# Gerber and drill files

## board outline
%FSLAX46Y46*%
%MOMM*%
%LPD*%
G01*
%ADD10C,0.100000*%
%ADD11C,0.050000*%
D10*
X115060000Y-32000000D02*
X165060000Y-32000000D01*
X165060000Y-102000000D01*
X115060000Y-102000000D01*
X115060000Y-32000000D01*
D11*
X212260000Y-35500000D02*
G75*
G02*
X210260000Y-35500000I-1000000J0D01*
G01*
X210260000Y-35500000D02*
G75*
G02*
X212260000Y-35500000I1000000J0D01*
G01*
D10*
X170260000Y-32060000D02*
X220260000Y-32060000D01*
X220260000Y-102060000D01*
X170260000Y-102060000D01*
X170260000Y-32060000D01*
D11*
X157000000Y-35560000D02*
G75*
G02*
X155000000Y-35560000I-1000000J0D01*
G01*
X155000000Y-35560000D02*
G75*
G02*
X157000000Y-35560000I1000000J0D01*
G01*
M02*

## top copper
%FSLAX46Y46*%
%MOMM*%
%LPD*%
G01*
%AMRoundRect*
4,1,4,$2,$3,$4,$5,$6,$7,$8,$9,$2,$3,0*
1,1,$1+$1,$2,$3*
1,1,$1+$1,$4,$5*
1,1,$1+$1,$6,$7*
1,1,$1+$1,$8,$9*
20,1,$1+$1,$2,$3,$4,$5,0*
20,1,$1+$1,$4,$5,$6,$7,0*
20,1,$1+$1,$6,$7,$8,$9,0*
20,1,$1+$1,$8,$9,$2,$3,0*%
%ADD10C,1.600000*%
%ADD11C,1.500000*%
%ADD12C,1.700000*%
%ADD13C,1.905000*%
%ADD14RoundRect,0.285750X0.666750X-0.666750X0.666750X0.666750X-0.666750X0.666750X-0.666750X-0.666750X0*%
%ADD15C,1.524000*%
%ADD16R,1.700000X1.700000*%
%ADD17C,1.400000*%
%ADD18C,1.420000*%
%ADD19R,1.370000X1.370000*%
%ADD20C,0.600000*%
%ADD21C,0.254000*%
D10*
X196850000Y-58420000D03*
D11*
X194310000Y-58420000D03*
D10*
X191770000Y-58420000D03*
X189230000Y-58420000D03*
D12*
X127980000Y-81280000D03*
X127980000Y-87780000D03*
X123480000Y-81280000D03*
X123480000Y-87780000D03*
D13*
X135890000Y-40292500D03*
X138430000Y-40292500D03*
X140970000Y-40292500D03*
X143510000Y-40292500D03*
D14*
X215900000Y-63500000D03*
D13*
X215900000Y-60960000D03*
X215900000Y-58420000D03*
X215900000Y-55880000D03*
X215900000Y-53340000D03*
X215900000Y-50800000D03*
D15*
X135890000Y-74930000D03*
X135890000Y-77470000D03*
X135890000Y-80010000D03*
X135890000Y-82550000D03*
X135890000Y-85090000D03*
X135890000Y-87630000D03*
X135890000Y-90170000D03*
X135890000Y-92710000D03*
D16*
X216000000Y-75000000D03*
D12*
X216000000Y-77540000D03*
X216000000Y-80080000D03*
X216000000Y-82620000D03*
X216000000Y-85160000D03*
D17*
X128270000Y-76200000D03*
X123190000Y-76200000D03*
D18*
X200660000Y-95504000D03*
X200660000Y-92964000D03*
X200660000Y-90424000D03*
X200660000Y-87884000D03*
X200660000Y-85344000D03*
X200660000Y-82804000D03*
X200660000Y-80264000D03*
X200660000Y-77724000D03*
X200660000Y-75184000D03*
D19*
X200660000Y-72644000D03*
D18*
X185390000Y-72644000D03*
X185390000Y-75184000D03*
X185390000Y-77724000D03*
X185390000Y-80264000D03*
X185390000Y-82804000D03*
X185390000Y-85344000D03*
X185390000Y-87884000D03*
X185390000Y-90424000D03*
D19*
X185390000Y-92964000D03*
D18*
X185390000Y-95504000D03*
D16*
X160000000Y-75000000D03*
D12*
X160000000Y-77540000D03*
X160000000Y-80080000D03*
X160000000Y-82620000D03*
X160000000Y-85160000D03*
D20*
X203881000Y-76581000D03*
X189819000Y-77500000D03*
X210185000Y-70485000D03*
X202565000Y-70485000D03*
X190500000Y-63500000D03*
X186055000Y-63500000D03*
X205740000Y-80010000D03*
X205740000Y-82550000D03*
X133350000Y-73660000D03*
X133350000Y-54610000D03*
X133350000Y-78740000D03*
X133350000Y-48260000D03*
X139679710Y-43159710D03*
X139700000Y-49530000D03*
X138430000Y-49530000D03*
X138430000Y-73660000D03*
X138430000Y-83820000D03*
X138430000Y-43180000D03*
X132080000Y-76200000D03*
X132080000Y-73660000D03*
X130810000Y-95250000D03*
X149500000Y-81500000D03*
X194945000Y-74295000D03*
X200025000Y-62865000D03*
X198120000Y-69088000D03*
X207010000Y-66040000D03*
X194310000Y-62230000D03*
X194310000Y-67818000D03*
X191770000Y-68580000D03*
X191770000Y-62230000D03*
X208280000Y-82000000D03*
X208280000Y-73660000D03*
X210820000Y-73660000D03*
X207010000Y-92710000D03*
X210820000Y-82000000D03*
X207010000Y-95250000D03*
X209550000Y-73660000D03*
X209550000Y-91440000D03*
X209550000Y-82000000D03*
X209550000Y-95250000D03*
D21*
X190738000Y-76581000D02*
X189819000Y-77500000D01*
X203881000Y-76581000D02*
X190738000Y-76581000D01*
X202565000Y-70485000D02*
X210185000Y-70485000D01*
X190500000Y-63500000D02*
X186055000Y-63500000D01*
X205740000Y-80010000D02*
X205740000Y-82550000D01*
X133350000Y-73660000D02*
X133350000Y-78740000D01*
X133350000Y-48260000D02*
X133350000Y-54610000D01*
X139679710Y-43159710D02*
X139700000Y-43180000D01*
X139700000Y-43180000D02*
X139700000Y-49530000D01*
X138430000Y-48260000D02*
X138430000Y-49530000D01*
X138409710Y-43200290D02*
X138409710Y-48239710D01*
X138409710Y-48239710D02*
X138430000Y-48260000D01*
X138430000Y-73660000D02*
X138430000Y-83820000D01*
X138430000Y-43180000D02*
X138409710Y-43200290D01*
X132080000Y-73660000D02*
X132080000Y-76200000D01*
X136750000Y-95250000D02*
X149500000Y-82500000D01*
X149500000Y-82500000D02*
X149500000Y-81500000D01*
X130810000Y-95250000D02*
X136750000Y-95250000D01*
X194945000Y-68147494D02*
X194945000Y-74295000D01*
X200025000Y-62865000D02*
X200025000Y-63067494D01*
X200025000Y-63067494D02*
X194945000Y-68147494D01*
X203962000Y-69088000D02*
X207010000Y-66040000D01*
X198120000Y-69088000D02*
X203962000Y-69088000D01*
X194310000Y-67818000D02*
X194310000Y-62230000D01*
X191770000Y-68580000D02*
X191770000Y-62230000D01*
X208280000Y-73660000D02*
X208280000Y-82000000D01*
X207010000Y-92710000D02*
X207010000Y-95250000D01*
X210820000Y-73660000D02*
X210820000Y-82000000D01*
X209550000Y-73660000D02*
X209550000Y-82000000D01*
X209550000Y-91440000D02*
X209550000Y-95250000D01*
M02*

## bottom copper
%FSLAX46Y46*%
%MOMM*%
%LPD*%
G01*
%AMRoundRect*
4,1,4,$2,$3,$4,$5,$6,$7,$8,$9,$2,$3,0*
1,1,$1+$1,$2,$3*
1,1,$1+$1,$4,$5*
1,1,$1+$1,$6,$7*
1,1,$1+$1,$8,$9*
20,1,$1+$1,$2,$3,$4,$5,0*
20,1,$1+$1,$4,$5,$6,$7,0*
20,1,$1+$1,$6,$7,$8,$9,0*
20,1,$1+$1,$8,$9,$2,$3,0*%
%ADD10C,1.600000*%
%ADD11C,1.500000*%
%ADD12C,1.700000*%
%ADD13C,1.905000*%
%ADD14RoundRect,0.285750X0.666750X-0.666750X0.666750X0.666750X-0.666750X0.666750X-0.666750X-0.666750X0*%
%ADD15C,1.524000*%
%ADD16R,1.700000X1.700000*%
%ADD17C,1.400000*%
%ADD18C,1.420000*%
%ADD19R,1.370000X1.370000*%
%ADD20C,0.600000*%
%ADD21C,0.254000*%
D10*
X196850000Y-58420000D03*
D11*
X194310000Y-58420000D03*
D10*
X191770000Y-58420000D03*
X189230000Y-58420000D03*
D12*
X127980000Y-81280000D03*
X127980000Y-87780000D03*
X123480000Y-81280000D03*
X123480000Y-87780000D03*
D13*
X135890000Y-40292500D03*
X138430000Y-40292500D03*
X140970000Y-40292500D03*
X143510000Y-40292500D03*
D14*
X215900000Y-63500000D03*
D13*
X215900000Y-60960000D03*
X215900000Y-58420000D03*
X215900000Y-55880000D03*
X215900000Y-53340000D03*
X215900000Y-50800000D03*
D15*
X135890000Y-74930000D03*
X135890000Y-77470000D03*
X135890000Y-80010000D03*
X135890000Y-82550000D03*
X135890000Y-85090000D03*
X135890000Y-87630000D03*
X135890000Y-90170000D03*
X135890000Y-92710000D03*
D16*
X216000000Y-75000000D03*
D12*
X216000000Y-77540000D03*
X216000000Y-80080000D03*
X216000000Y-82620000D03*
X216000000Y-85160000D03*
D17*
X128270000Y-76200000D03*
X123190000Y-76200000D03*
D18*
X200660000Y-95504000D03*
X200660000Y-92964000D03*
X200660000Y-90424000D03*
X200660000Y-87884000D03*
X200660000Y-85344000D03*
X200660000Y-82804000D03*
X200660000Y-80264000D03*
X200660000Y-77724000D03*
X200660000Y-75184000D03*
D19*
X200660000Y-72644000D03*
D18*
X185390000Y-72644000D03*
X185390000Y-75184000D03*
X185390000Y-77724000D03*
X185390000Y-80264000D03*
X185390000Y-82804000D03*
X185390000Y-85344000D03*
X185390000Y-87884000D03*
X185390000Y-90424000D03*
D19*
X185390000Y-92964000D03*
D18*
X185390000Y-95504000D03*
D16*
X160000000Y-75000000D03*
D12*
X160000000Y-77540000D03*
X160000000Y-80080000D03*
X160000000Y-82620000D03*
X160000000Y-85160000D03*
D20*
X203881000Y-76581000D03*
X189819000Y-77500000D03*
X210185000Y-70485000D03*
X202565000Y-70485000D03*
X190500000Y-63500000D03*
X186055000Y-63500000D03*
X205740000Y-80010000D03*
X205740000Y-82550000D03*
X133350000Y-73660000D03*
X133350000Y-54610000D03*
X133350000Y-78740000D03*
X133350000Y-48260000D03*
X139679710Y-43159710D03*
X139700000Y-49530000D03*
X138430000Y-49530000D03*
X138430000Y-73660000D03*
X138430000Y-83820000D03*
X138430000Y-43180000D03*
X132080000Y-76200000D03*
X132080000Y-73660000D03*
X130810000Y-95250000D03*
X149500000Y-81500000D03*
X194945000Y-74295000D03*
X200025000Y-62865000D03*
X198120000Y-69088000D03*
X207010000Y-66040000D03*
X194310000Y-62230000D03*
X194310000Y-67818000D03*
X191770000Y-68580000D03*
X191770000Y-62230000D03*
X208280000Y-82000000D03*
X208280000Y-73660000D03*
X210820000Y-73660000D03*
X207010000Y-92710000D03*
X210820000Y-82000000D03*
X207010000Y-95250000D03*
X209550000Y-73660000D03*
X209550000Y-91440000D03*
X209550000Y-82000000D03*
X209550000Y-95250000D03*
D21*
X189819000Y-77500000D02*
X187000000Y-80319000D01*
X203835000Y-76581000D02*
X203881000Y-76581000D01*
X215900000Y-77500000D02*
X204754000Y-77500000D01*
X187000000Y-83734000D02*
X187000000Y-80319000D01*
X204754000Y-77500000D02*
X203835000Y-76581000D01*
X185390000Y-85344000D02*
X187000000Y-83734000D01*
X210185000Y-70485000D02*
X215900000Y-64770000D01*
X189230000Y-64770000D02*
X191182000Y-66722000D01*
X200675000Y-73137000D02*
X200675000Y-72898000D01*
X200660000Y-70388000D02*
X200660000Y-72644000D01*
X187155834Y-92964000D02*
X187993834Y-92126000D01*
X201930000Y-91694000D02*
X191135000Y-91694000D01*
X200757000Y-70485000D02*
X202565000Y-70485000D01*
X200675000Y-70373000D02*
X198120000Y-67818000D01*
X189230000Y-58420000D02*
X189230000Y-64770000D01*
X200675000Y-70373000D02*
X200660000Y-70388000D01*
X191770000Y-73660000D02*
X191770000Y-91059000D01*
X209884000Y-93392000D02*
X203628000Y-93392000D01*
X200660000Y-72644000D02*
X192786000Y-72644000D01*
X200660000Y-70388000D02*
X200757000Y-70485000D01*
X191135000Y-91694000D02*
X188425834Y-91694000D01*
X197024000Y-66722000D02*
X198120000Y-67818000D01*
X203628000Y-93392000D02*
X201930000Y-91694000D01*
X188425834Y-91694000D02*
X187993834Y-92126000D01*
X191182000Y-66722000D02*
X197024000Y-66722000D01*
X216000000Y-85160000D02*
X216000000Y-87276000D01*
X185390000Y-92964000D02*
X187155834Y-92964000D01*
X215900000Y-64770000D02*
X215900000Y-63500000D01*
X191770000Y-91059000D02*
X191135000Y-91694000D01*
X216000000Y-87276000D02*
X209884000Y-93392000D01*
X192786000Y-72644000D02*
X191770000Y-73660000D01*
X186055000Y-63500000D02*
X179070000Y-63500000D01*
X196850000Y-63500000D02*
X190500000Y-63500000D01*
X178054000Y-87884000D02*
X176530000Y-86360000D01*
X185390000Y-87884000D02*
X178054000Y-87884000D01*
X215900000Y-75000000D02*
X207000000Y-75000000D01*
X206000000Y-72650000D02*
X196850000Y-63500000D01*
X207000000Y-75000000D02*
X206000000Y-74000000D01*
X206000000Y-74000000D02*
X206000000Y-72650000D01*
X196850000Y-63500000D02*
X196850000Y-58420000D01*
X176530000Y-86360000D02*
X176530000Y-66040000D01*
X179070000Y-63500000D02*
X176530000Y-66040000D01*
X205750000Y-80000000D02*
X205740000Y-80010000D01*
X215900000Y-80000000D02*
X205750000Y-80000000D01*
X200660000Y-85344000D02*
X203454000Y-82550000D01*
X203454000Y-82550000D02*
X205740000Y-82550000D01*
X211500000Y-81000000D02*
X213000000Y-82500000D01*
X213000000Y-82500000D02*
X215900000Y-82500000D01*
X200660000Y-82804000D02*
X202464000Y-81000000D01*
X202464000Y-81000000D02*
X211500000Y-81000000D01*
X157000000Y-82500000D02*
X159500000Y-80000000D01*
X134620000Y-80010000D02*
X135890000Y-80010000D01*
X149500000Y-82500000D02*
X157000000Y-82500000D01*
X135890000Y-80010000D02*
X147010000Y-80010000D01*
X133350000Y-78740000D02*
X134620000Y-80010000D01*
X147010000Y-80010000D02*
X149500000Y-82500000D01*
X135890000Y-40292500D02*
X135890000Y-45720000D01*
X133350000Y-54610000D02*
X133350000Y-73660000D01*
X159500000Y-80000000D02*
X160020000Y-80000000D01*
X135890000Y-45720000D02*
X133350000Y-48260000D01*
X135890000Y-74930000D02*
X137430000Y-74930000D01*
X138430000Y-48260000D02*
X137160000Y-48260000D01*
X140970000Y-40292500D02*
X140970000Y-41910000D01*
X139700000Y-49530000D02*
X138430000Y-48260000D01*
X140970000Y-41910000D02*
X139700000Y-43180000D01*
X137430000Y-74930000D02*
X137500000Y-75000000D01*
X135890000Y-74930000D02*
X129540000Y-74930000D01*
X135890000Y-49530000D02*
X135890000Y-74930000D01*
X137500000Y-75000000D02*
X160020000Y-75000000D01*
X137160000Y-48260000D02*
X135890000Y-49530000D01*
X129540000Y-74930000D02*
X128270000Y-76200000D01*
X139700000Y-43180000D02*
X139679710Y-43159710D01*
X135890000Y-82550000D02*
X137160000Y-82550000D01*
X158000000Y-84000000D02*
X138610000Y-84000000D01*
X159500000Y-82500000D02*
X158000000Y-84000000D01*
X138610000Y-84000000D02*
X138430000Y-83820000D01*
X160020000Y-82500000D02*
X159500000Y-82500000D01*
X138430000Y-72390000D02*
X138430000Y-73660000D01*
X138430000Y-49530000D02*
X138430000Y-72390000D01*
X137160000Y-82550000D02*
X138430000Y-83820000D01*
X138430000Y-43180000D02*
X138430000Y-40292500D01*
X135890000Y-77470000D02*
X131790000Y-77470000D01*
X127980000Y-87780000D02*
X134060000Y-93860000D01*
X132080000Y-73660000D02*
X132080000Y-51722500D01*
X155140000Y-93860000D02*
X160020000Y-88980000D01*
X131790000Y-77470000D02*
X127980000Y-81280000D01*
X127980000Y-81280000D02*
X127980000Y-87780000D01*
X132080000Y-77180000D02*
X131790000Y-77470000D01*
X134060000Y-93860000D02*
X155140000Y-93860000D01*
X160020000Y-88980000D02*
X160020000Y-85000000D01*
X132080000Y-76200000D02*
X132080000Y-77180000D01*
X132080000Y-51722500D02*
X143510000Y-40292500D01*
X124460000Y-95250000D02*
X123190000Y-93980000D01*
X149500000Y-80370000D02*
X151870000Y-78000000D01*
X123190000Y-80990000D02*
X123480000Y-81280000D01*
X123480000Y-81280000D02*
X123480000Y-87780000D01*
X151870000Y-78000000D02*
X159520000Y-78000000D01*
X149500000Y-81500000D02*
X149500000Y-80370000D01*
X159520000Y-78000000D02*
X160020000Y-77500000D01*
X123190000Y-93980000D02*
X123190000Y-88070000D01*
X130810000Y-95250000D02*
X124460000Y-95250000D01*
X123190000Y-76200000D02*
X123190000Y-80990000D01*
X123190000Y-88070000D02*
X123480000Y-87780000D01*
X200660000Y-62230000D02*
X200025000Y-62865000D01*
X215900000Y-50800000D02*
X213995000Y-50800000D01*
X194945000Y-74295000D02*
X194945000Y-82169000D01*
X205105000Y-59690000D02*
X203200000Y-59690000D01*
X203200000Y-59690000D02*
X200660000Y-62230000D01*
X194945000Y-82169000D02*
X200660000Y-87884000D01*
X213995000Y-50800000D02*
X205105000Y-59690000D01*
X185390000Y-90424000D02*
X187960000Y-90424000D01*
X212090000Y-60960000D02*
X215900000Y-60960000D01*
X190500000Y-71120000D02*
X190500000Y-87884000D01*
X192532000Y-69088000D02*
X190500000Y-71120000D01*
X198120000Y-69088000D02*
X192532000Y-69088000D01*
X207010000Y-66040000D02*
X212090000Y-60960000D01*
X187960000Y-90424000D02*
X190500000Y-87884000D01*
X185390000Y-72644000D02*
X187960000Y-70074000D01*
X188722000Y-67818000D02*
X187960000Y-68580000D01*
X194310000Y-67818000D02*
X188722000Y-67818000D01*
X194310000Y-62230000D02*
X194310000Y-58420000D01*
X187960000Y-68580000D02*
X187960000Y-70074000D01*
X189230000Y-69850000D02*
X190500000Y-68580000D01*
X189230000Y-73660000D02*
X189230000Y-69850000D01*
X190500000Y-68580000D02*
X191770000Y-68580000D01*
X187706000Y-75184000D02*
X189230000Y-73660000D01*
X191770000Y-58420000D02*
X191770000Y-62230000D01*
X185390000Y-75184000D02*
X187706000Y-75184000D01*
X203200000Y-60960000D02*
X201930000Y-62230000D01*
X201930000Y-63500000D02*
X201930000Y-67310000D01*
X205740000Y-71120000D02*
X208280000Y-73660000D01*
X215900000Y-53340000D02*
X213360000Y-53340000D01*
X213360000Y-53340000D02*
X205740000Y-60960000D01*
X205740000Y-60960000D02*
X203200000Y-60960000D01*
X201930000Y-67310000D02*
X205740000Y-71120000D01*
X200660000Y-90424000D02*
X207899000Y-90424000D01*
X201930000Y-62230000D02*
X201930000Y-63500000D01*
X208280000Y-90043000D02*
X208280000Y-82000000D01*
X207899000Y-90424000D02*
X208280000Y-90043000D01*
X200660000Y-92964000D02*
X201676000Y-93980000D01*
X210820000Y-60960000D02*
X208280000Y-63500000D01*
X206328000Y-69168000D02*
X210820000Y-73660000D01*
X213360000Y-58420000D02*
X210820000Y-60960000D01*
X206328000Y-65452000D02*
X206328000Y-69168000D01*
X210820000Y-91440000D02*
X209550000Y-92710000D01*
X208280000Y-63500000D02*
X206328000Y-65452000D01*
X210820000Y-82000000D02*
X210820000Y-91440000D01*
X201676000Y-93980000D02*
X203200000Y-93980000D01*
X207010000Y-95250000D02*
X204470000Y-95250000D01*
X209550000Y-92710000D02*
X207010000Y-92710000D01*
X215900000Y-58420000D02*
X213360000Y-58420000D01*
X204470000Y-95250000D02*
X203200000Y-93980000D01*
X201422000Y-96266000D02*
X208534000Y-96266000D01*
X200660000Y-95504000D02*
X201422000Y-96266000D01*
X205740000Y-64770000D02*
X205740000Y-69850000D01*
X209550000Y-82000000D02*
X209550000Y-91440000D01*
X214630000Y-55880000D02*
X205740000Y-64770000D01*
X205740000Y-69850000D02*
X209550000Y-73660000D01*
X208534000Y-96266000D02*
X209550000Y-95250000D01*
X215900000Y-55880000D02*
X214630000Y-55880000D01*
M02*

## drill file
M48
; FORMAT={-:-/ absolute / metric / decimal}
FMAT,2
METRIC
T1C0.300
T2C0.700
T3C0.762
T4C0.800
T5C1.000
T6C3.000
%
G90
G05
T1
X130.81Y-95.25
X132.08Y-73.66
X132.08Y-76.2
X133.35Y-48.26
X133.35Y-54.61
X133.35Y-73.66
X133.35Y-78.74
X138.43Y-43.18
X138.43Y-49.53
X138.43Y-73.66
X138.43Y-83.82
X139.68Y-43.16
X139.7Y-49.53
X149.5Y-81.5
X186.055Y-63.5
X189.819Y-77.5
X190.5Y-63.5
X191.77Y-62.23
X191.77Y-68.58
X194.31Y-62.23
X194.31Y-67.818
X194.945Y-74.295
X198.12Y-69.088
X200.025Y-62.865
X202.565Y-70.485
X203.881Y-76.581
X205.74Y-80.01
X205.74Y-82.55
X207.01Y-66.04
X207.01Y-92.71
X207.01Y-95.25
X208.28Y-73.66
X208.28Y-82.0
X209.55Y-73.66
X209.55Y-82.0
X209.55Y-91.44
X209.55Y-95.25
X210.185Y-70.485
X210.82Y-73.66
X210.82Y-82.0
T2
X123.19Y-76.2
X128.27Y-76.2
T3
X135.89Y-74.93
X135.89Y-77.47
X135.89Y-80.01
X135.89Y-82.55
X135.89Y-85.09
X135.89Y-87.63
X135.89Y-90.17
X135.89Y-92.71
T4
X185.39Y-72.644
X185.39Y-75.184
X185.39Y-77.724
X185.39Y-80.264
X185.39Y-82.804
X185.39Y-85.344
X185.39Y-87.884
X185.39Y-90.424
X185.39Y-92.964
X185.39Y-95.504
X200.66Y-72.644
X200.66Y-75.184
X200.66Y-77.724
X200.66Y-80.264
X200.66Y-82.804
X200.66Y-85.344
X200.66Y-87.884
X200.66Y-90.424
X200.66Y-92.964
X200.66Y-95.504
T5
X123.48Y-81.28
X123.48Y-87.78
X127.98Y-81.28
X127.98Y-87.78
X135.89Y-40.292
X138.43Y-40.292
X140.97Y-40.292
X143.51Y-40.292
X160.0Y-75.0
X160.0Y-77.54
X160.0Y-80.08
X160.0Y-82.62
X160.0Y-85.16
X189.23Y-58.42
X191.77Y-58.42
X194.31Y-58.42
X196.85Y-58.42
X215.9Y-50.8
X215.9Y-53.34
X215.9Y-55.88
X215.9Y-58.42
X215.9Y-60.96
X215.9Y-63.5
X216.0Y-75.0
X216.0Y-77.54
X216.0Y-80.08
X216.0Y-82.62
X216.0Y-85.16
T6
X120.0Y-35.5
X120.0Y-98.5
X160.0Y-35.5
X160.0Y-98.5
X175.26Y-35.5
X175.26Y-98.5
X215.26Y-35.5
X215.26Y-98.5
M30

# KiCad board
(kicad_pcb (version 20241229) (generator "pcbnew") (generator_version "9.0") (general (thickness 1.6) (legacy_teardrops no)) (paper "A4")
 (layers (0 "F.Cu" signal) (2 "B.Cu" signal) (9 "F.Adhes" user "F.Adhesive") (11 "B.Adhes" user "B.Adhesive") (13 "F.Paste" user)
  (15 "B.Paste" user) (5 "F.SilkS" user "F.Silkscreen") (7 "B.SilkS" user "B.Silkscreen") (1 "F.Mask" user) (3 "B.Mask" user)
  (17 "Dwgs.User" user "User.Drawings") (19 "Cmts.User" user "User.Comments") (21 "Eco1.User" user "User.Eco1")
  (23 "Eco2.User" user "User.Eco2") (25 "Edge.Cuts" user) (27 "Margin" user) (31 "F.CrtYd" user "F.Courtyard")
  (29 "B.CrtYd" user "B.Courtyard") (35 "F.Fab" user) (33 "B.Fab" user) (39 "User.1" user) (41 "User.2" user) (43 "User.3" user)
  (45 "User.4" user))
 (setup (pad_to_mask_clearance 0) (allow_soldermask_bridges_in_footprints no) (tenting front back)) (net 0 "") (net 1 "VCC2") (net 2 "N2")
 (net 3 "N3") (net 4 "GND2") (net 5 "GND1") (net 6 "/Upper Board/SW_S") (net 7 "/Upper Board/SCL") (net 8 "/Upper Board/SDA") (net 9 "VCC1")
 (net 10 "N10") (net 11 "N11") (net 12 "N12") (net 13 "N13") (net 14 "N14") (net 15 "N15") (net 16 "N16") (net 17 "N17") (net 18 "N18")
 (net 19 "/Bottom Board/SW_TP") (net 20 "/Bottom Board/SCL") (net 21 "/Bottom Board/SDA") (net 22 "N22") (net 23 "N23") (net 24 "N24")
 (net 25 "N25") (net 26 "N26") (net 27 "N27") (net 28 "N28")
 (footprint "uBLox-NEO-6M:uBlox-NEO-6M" (layer "F.Cu") (at 193.04 43.18 180)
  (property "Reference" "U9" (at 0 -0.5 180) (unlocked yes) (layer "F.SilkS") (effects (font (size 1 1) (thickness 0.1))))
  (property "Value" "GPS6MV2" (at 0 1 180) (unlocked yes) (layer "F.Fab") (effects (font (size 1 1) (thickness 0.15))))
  (pad "1" thru_hole circle (at -3.81 -15.24 180) (size 1.6 1.6) (drill 1) (layers "*.Cu" "*.Mask") (remove_unused_layers no) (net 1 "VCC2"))
  (pad "2" thru_hole circle (at -1.27 -15.24 180) (size 1.5 1.5) (drill 1) (layers "*.Cu" "F.Mask" "F.Paste") (remove_unused_layers no)
   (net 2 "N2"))
  (pad "3" thru_hole circle (at 1.27 -15.24 180) (size 1.6 1.6) (drill 1) (layers "*.Cu" "F.Mask" "F.Paste") (remove_unused_layers no)
   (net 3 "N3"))
  (pad "4" thru_hole circle (at 3.81 -15.24 180) (size 1.6 1.6) (drill 1) (layers "*.Cu" "F.Mask" "F.Paste") (remove_unused_layers no)
   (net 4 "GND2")))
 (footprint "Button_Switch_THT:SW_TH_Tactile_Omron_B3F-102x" (layer "F.Cu") (at 127.98 81.28 -90)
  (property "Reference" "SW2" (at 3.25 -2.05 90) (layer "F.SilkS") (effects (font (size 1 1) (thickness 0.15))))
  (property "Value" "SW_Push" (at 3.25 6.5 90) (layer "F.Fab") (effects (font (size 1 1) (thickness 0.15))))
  (pad "1" thru_hole circle (at 0 0 270) (size 1.7 1.7) (drill 1) (layers "*.Cu" "*.Mask") (remove_unused_layers no) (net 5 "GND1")
   (thermal_bridge_angle 90))
  (pad "1" thru_hole circle (at 6.5 0 270) (size 1.7 1.7) (drill 1) (layers "*.Cu" "*.Mask") (remove_unused_layers no) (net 5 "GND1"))
  (pad "2" thru_hole circle (at 0 4.5 270) (size 1.7 1.7) (drill 1) (layers "*.Cu" "*.Mask") (remove_unused_layers no)
   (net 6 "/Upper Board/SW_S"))
  (pad "2" thru_hole circle (at 6.5 4.5 270) (size 1.7 1.7) (drill 1) (layers "*.Cu" "*.Mask") (remove_unused_layers no)
   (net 6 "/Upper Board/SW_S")))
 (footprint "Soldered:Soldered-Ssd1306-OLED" (layer "F.Cu") (at 139.7 40.2925)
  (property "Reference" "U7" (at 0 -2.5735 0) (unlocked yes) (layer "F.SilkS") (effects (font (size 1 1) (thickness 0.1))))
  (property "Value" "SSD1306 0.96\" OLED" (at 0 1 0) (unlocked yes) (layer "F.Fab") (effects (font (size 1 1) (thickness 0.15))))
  (pad "1" thru_hole circle (at -3.81 0) (size 1.905 1.905) (drill 1) (layers "*.Cu" "*.Mask") (remove_unused_layers no)
   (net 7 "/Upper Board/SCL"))
  (pad "2" thru_hole circle (at -1.27 0) (size 1.905 1.905) (drill 1) (layers "*.Cu" "*.Mask") (remove_unused_layers no)
   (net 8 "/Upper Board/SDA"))
  (pad "3" thru_hole circle (at 1.27 0) (size 1.905 1.905) (drill 1) (layers "*.Cu" "*.Mask") (remove_unused_layers no) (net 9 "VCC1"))
  (pad "4" thru_hole circle (at 3.81 0) (size 1.905 1.905) (drill 1) (layers "*.Cu" "*.Mask") (remove_unused_layers no) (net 5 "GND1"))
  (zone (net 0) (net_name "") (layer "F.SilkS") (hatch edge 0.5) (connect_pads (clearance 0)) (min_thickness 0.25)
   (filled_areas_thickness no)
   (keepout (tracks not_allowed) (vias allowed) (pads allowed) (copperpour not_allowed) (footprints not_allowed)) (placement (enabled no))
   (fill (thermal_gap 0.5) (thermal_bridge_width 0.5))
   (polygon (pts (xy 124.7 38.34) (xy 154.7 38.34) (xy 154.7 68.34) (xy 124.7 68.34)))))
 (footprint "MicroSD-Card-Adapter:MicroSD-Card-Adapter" (layer "F.Cu") (at 215.9 57.2008 90)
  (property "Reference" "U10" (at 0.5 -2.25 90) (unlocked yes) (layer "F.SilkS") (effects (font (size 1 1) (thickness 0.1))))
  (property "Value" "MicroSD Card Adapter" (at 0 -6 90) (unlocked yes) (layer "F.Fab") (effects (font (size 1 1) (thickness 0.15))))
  (pad "1" thru_hole roundrect (at -6.2992 0 90) (size 1.905 1.905) (drill 1) (layers "*.Cu" "*.Mask") (remove_unused_layers no)
   (roundrect_rratio 0.15) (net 4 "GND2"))
  (pad "2" thru_hole circle (at -3.7592 0 90) (size 1.905 1.905) (drill 1) (layers "*.Cu" "*.Mask") (remove_unused_layers no) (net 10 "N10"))
  (pad "3" thru_hole circle (at -1.2192 0 90) (size 1.905 1.905) (drill 1) (layers "*.Cu" "*.Mask") (remove_unused_layers no) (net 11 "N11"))
  (pad "4" thru_hole circle (at 1.3208 0 90) (size 1.905 1.905) (drill 1) (layers "*.Cu" "*.Mask") (remove_unused_layers no) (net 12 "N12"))
  (pad "5" thru_hole circle (at 3.8608 0 90) (size 1.905 1.905) (drill 1) (layers "*.Cu" "*.Mask") (remove_unused_layers no) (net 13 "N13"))
  (pad "6" thru_hole circle (at 6.4008 0 90) (size 1.905 1.905) (drill 1) (layers "*.Cu" "*.Mask") (remove_unused_layers no) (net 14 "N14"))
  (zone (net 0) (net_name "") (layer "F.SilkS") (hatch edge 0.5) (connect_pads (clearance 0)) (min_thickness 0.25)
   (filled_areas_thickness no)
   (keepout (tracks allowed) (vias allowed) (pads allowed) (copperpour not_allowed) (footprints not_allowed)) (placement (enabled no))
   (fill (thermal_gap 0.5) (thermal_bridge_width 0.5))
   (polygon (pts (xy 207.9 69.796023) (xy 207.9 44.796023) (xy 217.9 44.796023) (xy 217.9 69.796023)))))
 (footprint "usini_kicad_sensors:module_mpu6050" (layer "F.Cu") (at 135.89 92.71)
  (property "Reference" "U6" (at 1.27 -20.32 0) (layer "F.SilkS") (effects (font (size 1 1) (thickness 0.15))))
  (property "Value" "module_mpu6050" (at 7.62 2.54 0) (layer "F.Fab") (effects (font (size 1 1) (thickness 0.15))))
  (pad "1" thru_hole circle (at 0 -17.78) (size 1.524 1.524) (drill 0.762) (layers "*.Cu" "*.Mask") (remove_unused_layers no) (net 9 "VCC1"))
  (pad "2" thru_hole circle (at 0 -15.24) (size 1.524 1.524) (drill 0.762) (layers "*.Cu" "*.Mask") (remove_unused_layers no) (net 5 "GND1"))
  (pad "3" thru_hole circle (at 0 -12.7) (size 1.524 1.524) (drill 0.762) (layers "*.Cu" "*.Mask") (remove_unused_layers no)
   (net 7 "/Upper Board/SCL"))
  (pad "4" thru_hole circle (at 0 -10.16) (size 1.524 1.524) (drill 0.762) (layers "*.Cu" "*.Mask") (remove_unused_layers no)
   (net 8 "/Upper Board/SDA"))
  (pad "5" thru_hole circle (at 0 -7.62) (size 1.524 1.524) (drill 0.762) (layers "*.Cu" "*.Mask") (remove_unused_layers no) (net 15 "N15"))
  (pad "6" thru_hole circle (at 0 -5.08) (size 1.524 1.524) (drill 0.762) (layers "*.Cu" "*.Mask") (remove_unused_layers no) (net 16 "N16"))
  (pad "7" thru_hole circle (at 0 -2.54) (size 1.524 1.524) (drill 0.762) (layers "*.Cu" "*.Mask") (remove_unused_layers no) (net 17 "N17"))
  (pad "8" thru_hole circle (at 0 0) (size 1.524 1.524) (drill 0.762) (layers "*.Cu" "*.Mask") (remove_unused_layers no) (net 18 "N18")))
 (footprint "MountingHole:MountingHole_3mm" (layer "F.Cu") (at 215.26 98.5)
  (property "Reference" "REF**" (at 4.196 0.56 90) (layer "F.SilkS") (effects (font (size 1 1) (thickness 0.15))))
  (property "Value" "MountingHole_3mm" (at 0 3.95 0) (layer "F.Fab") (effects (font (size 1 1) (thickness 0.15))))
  (pad "" np_thru_hole circle (at 0 0) (size 3 3) (drill 3) (layers "*.Cu" "*.Mask")))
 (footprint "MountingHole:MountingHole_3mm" (layer "F.Cu") (at 160 98.5)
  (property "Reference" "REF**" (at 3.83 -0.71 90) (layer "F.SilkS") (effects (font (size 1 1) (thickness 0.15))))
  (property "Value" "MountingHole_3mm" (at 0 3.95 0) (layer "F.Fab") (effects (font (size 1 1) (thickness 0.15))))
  (pad "" np_thru_hole circle (at 0 0) (size 3 3) (drill 3) (layers "*.Cu" "*.Mask")))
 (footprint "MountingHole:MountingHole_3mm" (layer "F.Cu") (at 175.26 98.5)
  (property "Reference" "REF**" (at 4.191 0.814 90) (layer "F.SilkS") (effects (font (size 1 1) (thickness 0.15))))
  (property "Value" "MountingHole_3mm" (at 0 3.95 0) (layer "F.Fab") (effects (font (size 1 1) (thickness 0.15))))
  (pad "" np_thru_hole circle (at 0 0) (size 3 3) (drill 3) (layers "*.Cu" "*.Mask")))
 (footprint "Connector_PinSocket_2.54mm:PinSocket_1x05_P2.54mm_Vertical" (layer "F.Cu") (at 216 75)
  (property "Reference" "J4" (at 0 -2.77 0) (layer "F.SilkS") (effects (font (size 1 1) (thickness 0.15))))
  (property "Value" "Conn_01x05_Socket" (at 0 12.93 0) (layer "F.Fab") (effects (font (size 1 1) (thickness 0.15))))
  (pad "1" thru_hole rect (at 0 0) (size 1.7 1.7) (drill 1) (layers "*.Cu" "*.Mask") (remove_unused_layers no) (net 1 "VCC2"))
  (pad "2" thru_hole circle (at 0 2.54) (size 1.7 1.7) (drill 1) (layers "*.Cu" "*.Mask") (remove_unused_layers no)
   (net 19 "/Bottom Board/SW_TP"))
  (pad "3" thru_hole circle (at 0 5.08) (size 1.7 1.7) (drill 1) (layers "*.Cu" "*.Mask") (remove_unused_layers no)
   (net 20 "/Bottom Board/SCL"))
  (pad "4" thru_hole circle (at 0 7.62) (size 1.7 1.7) (drill 1) (layers "*.Cu" "*.Mask") (remove_unused_layers no)
   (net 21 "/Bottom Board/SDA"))
  (pad "5" thru_hole circle (at 0 10.16) (size 1.7 1.7) (drill 1) (layers "*.Cu" "*.Mask") (remove_unused_layers no) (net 4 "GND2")))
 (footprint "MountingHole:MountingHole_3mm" (layer "F.Cu") (at 215.26 35.5)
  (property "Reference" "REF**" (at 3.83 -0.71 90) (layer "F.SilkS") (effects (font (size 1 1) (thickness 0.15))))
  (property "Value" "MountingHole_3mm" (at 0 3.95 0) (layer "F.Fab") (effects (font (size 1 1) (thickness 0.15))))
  (pad "" np_thru_hole circle (at 0 0) (size 3 3) (drill 3) (layers "*.Cu" "*.Mask")))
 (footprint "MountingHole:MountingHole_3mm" (layer "F.Cu") (at 120 35.5)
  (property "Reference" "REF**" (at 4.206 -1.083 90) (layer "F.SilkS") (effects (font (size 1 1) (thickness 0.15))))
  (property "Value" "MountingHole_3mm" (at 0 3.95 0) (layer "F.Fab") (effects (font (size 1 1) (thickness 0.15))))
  (pad "" np_thru_hole circle (at 0 0) (size 3 3) (drill 3) (layers "*.Cu" "*.Mask")))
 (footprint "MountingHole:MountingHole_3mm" (layer "F.Cu") (at 175.26 35.5)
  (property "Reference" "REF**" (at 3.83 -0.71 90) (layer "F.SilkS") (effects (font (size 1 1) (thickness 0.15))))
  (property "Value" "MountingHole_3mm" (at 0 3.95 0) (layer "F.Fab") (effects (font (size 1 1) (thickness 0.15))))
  (pad "" np_thru_hole circle (at 0 0) (size 3 3) (drill 3) (layers "*.Cu" "*.Mask")))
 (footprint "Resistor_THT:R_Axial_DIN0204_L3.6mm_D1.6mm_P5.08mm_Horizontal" (layer "F.Cu") (at 128.27 76.2 180)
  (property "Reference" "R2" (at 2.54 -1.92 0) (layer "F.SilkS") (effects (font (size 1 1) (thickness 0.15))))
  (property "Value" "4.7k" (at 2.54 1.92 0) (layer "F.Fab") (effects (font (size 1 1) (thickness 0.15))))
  (pad "1" thru_hole circle (at 0 0 180) (size 1.4 1.4) (drill 0.7) (layers "*.Cu" "*.Mask") (remove_unused_layers no) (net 9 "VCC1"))
  (pad "2" thru_hole circle (at 5.08 0 180) (size 1.4 1.4) (drill 0.7) (layers "*.Cu" "*.Mask") (remove_unused_layers no)
   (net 6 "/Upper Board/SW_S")))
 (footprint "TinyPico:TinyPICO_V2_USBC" (layer "F.Cu") (at 193.025 84.074 180)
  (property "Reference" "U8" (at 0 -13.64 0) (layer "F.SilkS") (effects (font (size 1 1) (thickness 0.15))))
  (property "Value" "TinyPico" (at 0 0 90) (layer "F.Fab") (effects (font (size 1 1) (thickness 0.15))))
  (pad "1" thru_hole circle (at -7.635 -11.43 90) (size 1.42 1.42) (drill 0.8) (layers "*.Cu" "*.Mask") (remove_unused_layers no)
   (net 12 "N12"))
  (pad "2" thru_hole circle (at -7.635 -8.89 90) (size 1.42 1.42) (drill 0.8) (layers "*.Cu" "*.Mask") (remove_unused_layers no)
   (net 11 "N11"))
  (pad "3" thru_hole circle (at -7.635 -6.35 90) (size 1.42 1.42) (drill 0.8) (layers "*.Cu" "*.Mask") (remove_unused_layers no)
   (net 13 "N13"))
  (pad "4" thru_hole circle (at -7.635 -3.81 90) (size 1.42 1.42) (drill 0.8) (layers "*.Cu" "*.Mask") (remove_unused_layers no)
   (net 14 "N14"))
  (pad "5" thru_hole circle (at -7.635 -1.27 90) (size 1.42 1.42) (drill 0.8) (layers "*.Cu" "*.Mask") (remove_unused_layers no)
   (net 20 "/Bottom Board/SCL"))
  (pad "6" thru_hole circle (at -7.635 1.27 90) (size 1.42 1.42) (drill 0.8) (layers "*.Cu" "*.Mask") (remove_unused_layers no)
   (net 21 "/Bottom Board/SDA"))
  (pad "7" thru_hole circle (at -7.635 3.81 90) (size 1.42 1.42) (drill 0.8) (layers "*.Cu" "*.Mask") (remove_unused_layers no)
   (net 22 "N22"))
  (pad "8" thru_hole circle (at -7.635 6.35 90) (size 1.42 1.42) (drill 0.8) (layers "*.Cu" "*.Mask") (remove_unused_layers no)
   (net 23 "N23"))
  (pad "9" thru_hole circle (at -7.635 8.89 90) (size 1.42 1.42) (drill 0.8) (layers "*.Cu" "*.Mask") (remove_unused_layers no)
   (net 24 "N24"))
  (pad "10" thru_hole rect (at -7.635 11.43 90) (size 1.37 1.37) (drill 0.8) (layers "*.Cu" "*.Mask") (remove_unused_layers no)
   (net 4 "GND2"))
  (pad "11" thru_hole circle (at 7.635 11.43 90) (size 1.42 1.42) (drill 0.8) (layers "*.Cu" "*.Mask") (remove_unused_layers no)
   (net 2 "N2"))
  (pad "12" thru_hole circle (at 7.635 8.89 90) (size 1.42 1.42) (drill 0.8) (layers "*.Cu" "*.Mask") (remove_unused_layers no) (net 3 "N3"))
  (pad "13" thru_hole circle (at 7.635 6.35 90) (size 1.42 1.42) (drill 0.8) (layers "*.Cu" "*.Mask") (remove_unused_layers no)
   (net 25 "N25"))
  (pad "14" thru_hole circle (at 7.635 3.81 90) (size 1.42 1.42) (drill 0.8) (layers "*.Cu" "*.Mask") (remove_unused_layers no)
   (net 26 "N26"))
  (pad "15" thru_hole circle (at 7.635 1.27 90) (size 1.42 1.42) (drill 0.8) (layers "*.Cu" "*.Mask") (remove_unused_layers no)
   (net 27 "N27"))
  (pad "16" thru_hole circle (at 7.635 -1.27 90) (size 1.42 1.42) (drill 0.8) (layers "*.Cu" "*.Mask") (remove_unused_layers no)
   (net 19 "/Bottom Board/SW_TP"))
  (pad "17" thru_hole circle (at 7.635 -3.81 90) (size 1.42 1.42) (drill 0.8) (layers "*.Cu" "*.Mask") (remove_unused_layers no)
   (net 1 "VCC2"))
  (pad "18" thru_hole circle (at 7.635 -6.35 90) (size 1.42 1.42) (drill 0.8) (layers "*.Cu" "*.Mask") (remove_unused_layers no)
   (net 10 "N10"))
  (pad "19" thru_hole rect (at 7.635 -8.89 90) (size 1.37 1.37) (drill 0.8) (layers "*.Cu" "*.Mask") (remove_unused_layers no)
   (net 4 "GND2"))
  (pad "20" thru_hole circle (at 7.635 -11.43 90) (size 1.42 1.42) (drill 0.8) (layers "*.Cu" "*.Mask") (remove_unused_layers no)
   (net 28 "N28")))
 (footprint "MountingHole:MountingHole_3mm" (layer "F.Cu") (at 120 98.5)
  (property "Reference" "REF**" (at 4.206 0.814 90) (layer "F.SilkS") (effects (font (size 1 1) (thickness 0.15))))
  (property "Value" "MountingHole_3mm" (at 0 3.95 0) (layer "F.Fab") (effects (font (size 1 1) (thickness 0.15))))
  (pad "" np_thru_hole circle (at 0 0) (size 3 3) (drill 3) (layers "*.Cu" "*.Mask")))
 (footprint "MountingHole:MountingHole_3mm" (layer "F.Cu") (at 160 35.5)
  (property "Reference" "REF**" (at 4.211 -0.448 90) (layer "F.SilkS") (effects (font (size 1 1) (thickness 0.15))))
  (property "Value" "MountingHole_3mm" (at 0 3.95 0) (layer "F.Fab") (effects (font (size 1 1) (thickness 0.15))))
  (pad "" np_thru_hole circle (at 0 0) (size 3 3) (drill 3) (layers "*.Cu" "*.Mask")))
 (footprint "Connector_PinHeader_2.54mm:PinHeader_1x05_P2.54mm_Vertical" (layer "B.Cu") (at 160 75 180)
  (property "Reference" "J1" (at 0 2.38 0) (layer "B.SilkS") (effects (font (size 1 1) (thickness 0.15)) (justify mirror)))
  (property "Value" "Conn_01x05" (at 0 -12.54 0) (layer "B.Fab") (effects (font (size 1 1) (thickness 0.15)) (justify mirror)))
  (pad "1" thru_hole rect (at 0 0 180) (size 1.7 1.7) (drill 1) (layers "*.Cu" "*.Mask") (remove_unused_layers no) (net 9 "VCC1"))
  (pad "2" thru_hole circle (at 0 -2.54 180) (size 1.7 1.7) (drill 1) (layers "*.Cu" "*.Mask") (remove_unused_layers no)
   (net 6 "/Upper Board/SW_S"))
  (pad "3" thru_hole circle (at 0 -5.08 180) (size 1.7 1.7) (drill 1) (layers "*.Cu" "*.Mask") (remove_unused_layers no)
   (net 7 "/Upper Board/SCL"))
  (pad "4" thru_hole circle (at 0 -7.62 180) (size 1.7 1.7) (drill 1) (layers "*.Cu" "*.Mask") (remove_unused_layers no)
   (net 8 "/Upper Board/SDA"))
  (pad "5" thru_hole circle (at 0 -10.16 180) (size 1.7 1.7) (drill 1) (layers "*.Cu" "*.Mask") (remove_unused_layers no) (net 5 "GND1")))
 (gr_rect (start 115.06 32) (end 165.06 102) (stroke (width 0.1) (type solid)) (fill no) (layer "Edge.Cuts"))
 (gr_circle (center 211.26 35.5) (end 212.26 35.5) (stroke (width 0.05) (type solid)) (fill no) (layer "Edge.Cuts"))
 (gr_rect (start 170.26 32.06) (end 220.26 102.06) (stroke (width 0.1) (type solid)) (fill no) (layer "Edge.Cuts"))
 (gr_circle (center 156 35.56) (end 157 35.56) (stroke (width 0.05) (type solid)) (fill no) (layer "Edge.Cuts"))
 (segment (start 190.738 76.581) (end 189.819 77.5) (width 0.254) (layer "F.Cu") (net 19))
 (segment (start 203.881 76.581) (end 190.738 76.581) (width 0.254) (layer "F.Cu") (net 19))
 (via (at 203.881 76.581) (size 0.6) (drill 0.3) (layers "F.Cu" "B.Cu") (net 19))
 (via (at 189.819 77.5) (size 0.6) (drill 0.3) (layers "F.Cu" "B.Cu") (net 19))
 (segment (start 189.819 77.5) (end 187 80.319) (width 0.254) (layer "B.Cu") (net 19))
 (segment (start 203.835 76.581) (end 203.881 76.581) (width 0.254) (layer "B.Cu") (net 19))
 (segment (start 215.9 77.5) (end 204.754 77.5) (width 0.254) (layer "B.Cu") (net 19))
 (segment (start 187 83.734) (end 187 80.319) (width 0.254) (layer "B.Cu") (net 19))
 (segment (start 204.754 77.5) (end 203.835 76.581) (width 0.254) (layer "B.Cu") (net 19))
 (segment (start 185.39 85.344) (end 187 83.734) (width 0.254) (layer "B.Cu") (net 19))
 (segment (start 202.565 70.485) (end 210.185 70.485) (width 0.254) (layer "F.Cu") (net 4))
 (via (at 210.185 70.485) (size 0.6) (drill 0.3) (layers "F.Cu" "B.Cu") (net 4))
 (via (at 202.565 70.485) (size 0.6) (drill 0.3) (layers "F.Cu" "B.Cu") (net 4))
 (segment (start 210.185 70.485) (end 215.9 64.77) (width 0.254) (layer "B.Cu") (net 4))
 (segment (start 189.23 64.77) (end 191.182 66.722) (width 0.254) (layer "B.Cu") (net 4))
 (segment (start 200.675 73.137) (end 200.675 72.898) (width 0.254) (layer "B.Cu") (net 4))
 (segment (start 200.66 70.388) (end 200.66 72.644) (width 0.254) (layer "B.Cu") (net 4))
 (segment (start 187.155834 92.964) (end 187.993834 92.126) (width 0.254) (layer "B.Cu") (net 4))
 (segment (start 201.93 91.694) (end 191.135 91.694) (width 0.254) (layer "B.Cu") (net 4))
 (segment (start 200.757 70.485) (end 202.565 70.485) (width 0.254) (layer "B.Cu") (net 4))
 (segment (start 200.675 70.373) (end 198.12 67.818) (width 0.254) (layer "B.Cu") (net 4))
 (segment (start 189.23 58.42) (end 189.23 64.77) (width 0.254) (layer "B.Cu") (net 4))
 (segment (start 200.675 70.373) (end 200.66 70.388) (width 0.254) (layer "B.Cu") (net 4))
 (segment (start 191.77 73.66) (end 191.77 91.059) (width 0.254) (layer "B.Cu") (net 4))
 (segment (start 209.884 93.392) (end 203.628 93.392) (width 0.254) (layer "B.Cu") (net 4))
 (segment (start 200.66 72.644) (end 192.786 72.644) (width 0.254) (layer "B.Cu") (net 4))
 (segment (start 200.66 70.388) (end 200.757 70.485) (width 0.254) (layer "B.Cu") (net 4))
 (segment (start 191.135 91.694) (end 188.425834 91.694) (width 0.254) (layer "B.Cu") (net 4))
 (segment (start 197.024 66.722) (end 198.12 67.818) (width 0.254) (layer "B.Cu") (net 4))
 (segment (start 203.628 93.392) (end 201.93 91.694) (width 0.254) (layer "B.Cu") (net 4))
 (segment (start 188.425834 91.694) (end 187.993834 92.126) (width 0.254) (layer "B.Cu") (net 4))
 (segment (start 191.182 66.722) (end 197.024 66.722) (width 0.254) (layer "B.Cu") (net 4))
 (segment (start 216 85.16) (end 216 87.276) (width 0.254) (layer "B.Cu") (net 4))
 (segment (start 185.39 92.964) (end 187.155834 92.964) (width 0.254) (layer "B.Cu") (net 4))
 (segment (start 215.9 64.77) (end 215.9 63.5) (width 0.254) (layer "B.Cu") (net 4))
 (segment (start 191.77 91.059) (end 191.135 91.694) (width 0.254) (layer "B.Cu") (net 4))
 (segment (start 216 87.276) (end 209.884 93.392) (width 0.254) (layer "B.Cu") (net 4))
 (segment (start 192.786 72.644) (end 191.77 73.66) (width 0.254) (layer "B.Cu") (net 4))
 (segment (start 190.5 63.5) (end 186.055 63.5) (width 0.254) (layer "F.Cu") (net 1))
 (via (at 190.5 63.5) (size 0.6) (drill 0.3) (layers "F.Cu" "B.Cu") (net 1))
 (via (at 186.055 63.5) (size 0.6) (drill 0.3) (layers "F.Cu" "B.Cu") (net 1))
 (segment (start 186.055 63.5) (end 179.07 63.5) (width 0.254) (layer "B.Cu") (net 1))
 (segment (start 196.85 63.5) (end 190.5 63.5) (width 0.254) (layer "B.Cu") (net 1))
 (segment (start 178.054 87.884) (end 176.53 86.36) (width 0.254) (layer "B.Cu") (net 1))
 (segment (start 185.39 87.884) (end 178.054 87.884) (width 0.254) (layer "B.Cu") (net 1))
 (segment (start 215.9 75) (end 207 75) (width 0.254) (layer "B.Cu") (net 1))
 (segment (start 206 72.65) (end 196.85 63.5) (width 0.254) (layer "B.Cu") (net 1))
 (segment (start 207 75) (end 206 74) (width 0.254) (layer "B.Cu") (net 1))
 (segment (start 206 74) (end 206 72.65) (width 0.254) (layer "B.Cu") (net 1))
 (segment (start 196.85 63.5) (end 196.85 58.42) (width 0.254) (layer "B.Cu") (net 1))
 (segment (start 176.53 86.36) (end 176.53 66.04) (width 0.254) (layer "B.Cu") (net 1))
 (segment (start 179.07 63.5) (end 176.53 66.04) (width 0.254) (layer "B.Cu") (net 1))
 (segment (start 205.74 80.01) (end 205.74 82.55) (width 0.254) (layer "F.Cu") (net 20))
 (via (at 205.74 80.01) (size 0.6) (drill 0.3) (layers "F.Cu" "B.Cu") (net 20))
 (via (at 205.74 82.55) (size 0.6) (drill 0.3) (layers "F.Cu" "B.Cu") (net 20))
 (segment (start 205.75 80) (end 205.74 80.01) (width 0.254) (layer "B.Cu") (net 20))
 (segment (start 215.9 80) (end 205.75 80) (width 0.254) (layer "B.Cu") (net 20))
 (segment (start 200.66 85.344) (end 203.454 82.55) (width 0.254) (layer "B.Cu") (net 20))
 (segment (start 203.454 82.55) (end 205.74 82.55) (width 0.254) (layer "B.Cu") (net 20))
 (segment (start 211.5 81) (end 213 82.5) (width 0.254) (layer "B.Cu") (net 21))
 (segment (start 213 82.5) (end 215.9 82.5) (width 0.254) (layer "B.Cu") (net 21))
 (segment (start 200.66 82.804) (end 202.464 81) (width 0.254) (layer "B.Cu") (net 21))
 (segment (start 202.464 81) (end 211.5 81) (width 0.254) (layer "B.Cu") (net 21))
 (segment (start 133.35 73.66) (end 133.35 78.74) (width 0.254) (layer "F.Cu") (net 7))
 (segment (start 133.35 48.26) (end 133.35 54.61) (width 0.254) (layer "F.Cu") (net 7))
 (via (at 133.35 73.66) (size 0.6) (drill 0.3) (layers "F.Cu" "B.Cu") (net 7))
 (via (at 133.35 54.61) (size 0.6) (drill 0.3) (layers "F.Cu" "B.Cu") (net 7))
 (via (at 133.35 78.74) (size 0.6) (drill 0.3) (layers "F.Cu" "B.Cu") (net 7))
 (via (at 133.35 48.26) (size 0.6) (drill 0.3) (layers "F.Cu" "B.Cu") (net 7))
 (segment (start 157 82.5) (end 159.5 80) (width 0.254) (layer "B.Cu") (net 7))
 (segment (start 134.62 80.01) (end 135.89 80.01) (width 0.254) (layer "B.Cu") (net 7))
 (segment (start 149.5 82.5) (end 157 82.5) (width 0.254) (layer "B.Cu") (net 7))
 (segment (start 135.89 80.01) (end 147.01 80.01) (width 0.254) (layer "B.Cu") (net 7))
 (segment (start 133.35 78.74) (end 134.62 80.01) (width 0.254) (layer "B.Cu") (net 7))
 (segment (start 147.01 80.01) (end 149.5 82.5) (width 0.254) (layer "B.Cu") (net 7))
 (segment (start 135.89 40.2925) (end 135.89 45.72) (width 0.254) (layer "B.Cu") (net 7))
 (segment (start 133.35 54.61) (end 133.35 73.66) (width 0.254) (layer "B.Cu") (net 7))
 (segment (start 159.5 80) (end 160.02 80) (width 0.254) (layer "B.Cu") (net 7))
 (segment (start 135.89 45.72) (end 133.35 48.26) (width 0.254) (layer "B.Cu") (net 7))
 (segment (start 139.67971 43.15971) (end 139.7 43.18) (width 0.254) (layer "F.Cu") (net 9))
 (segment (start 139.7 43.18) (end 139.7 49.53) (width 0.254) (layer "F.Cu") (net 9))
 (via (at 139.67971 43.15971) (size 0.6) (drill 0.3) (layers "F.Cu" "B.Cu") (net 9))
 (via (at 139.7 49.53) (size 0.6) (drill 0.3) (layers "F.Cu" "B.Cu") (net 9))
 (segment (start 135.89 74.93) (end 137.43 74.93) (width 0.254) (layer "B.Cu") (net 9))
 (segment (start 138.43 48.26) (end 137.16 48.26) (width 0.254) (layer "B.Cu") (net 9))
 (segment (start 140.97 40.2925) (end 140.97 41.91) (width 0.254) (layer "B.Cu") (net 9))
 (segment (start 139.7 49.53) (end 138.43 48.26) (width 0.254) (layer "B.Cu") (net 9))
 (segment (start 140.97 41.91) (end 139.7 43.18) (width 0.254) (layer "B.Cu") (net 9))
 (segment (start 137.43 74.93) (end 137.5 75) (width 0.254) (layer "B.Cu") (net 9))
 (segment (start 135.89 74.93) (end 129.54 74.93) (width 0.254) (layer "B.Cu") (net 9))
 (segment (start 135.89 49.53) (end 135.89 74.93) (width 0.254) (layer "B.Cu") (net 9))
 (segment (start 137.5 75) (end 160.02 75) (width 0.254) (layer "B.Cu") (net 9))
 (segment (start 137.16 48.26) (end 135.89 49.53) (width 0.254) (layer "B.Cu") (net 9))
 (segment (start 129.54 74.93) (end 128.27 76.2) (width 0.254) (layer "B.Cu") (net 9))
 (segment (start 139.7 43.18) (end 139.67971 43.15971) (width 0.254) (layer "B.Cu") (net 9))
 (segment (start 138.43 48.26) (end 138.43 49.53) (width 0.254) (layer "F.Cu") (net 8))
 (segment (start 138.40971 43.20029) (end 138.40971 48.23971) (width 0.254) (layer "F.Cu") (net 8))
 (segment (start 138.40971 48.23971) (end 138.43 48.26) (width 0.254) (layer "F.Cu") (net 8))
 (segment (start 138.43 73.66) (end 138.43 83.82) (width 0.254) (layer "F.Cu") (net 8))
 (segment (start 138.43 43.18) (end 138.40971 43.20029) (width 0.254) (layer "F.Cu") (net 8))
 (via (at 138.43 49.53) (size 0.6) (drill 0.3) (layers "F.Cu" "B.Cu") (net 8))
 (via (at 138.43 73.66) (size 0.6) (drill 0.3) (layers "F.Cu" "B.Cu") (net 8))
 (via (at 138.43 83.82) (size 0.6) (drill 0.3) (layers "F.Cu" "B.Cu") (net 8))
 (via (at 138.43 43.18) (size 0.6) (drill 0.3) (layers "F.Cu" "B.Cu") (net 8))
 (segment (start 135.89 82.55) (end 137.16 82.55) (width 0.254) (layer "B.Cu") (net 8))
 (segment (start 158 84) (end 138.61 84) (width 0.254) (layer "B.Cu") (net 8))
 (segment (start 159.5 82.5) (end 158 84) (width 0.254) (layer "B.Cu") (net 8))
 (segment (start 138.61 84) (end 138.43 83.82) (width 0.254) (layer "B.Cu") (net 8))
 (segment (start 160.02 82.5) (end 159.5 82.5) (width 0.254) (layer "B.Cu") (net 8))
 (segment (start 138.43 72.39) (end 138.43 73.66) (width 0.254) (layer "B.Cu") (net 8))
 (segment (start 138.43 49.53) (end 138.43 72.39) (width 0.254) (layer "B.Cu") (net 8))
 (segment (start 137.16 82.55) (end 138.43 83.82) (width 0.254) (layer "B.Cu") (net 8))
 (segment (start 138.43 43.18) (end 138.43 40.2925) (width 0.254) (layer "B.Cu") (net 8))
 (segment (start 132.08 73.66) (end 132.08 76.2) (width 0.254) (layer "F.Cu") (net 5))
 (via (at 132.08 76.2) (size 0.6) (drill 0.3) (layers "F.Cu" "B.Cu") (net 5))
 (via (at 132.08 73.66) (size 0.6) (drill 0.3) (layers "F.Cu" "B.Cu") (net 5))
 (segment (start 135.89 77.47) (end 131.79 77.47) (width 0.254) (layer "B.Cu") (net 5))
 (segment (start 127.98 87.78) (end 134.06 93.86) (width 0.254) (layer "B.Cu") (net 5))
 (segment (start 132.08 73.66) (end 132.08 51.7225) (width 0.254) (layer "B.Cu") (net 5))
 (segment (start 155.14 93.86) (end 160.02 88.98) (width 0.254) (layer "B.Cu") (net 5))
 (segment (start 131.79 77.47) (end 127.98 81.28) (width 0.254) (layer "B.Cu") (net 5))
 (segment (start 127.98 81.28) (end 127.98 87.78) (width 0.254) (layer "B.Cu") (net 5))
 (segment (start 132.08 77.18) (end 131.79 77.47) (width 0.254) (layer "B.Cu") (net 5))
 (segment (start 134.06 93.86) (end 155.14 93.86) (width 0.254) (layer "B.Cu") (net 5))
 (segment (start 160.02 88.98) (end 160.02 85) (width 0.254) (layer "B.Cu") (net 5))
 (segment (start 132.08 76.2) (end 132.08 77.18) (width 0.254) (layer "B.Cu") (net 5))
 (segment (start 132.08 51.7225) (end 143.51 40.2925) (width 0.254) (layer "B.Cu") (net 5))
 (segment (start 136.75 95.25) (end 149.5 82.5) (width 0.254) (layer "F.Cu") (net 6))
 (segment (start 149.5 82.5) (end 149.5 81.5) (width 0.254) (layer "F.Cu") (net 6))
 (segment (start 130.81 95.25) (end 136.75 95.25) (width 0.254) (layer "F.Cu") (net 6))
 (via (at 130.81 95.25) (size 0.6) (drill 0.3) (layers "F.Cu" "B.Cu") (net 6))
 (via (at 149.5 81.5) (size 0.6) (drill 0.3) (layers "F.Cu" "B.Cu") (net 6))
 (segment (start 124.46 95.25) (end 123.19 93.98) (width 0.254) (layer "B.Cu") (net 6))
 (segment (start 149.5 80.37) (end 151.87 78) (width 0.254) (layer "B.Cu") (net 6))
 (segment (start 123.19 80.99) (end 123.48 81.28) (width 0.254) (layer "B.Cu") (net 6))
 (segment (start 123.48 81.28) (end 123.48 87.78) (width 0.254) (layer "B.Cu") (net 6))
 (segment (start 151.87 78) (end 159.52 78) (width 0.254) (layer "B.Cu") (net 6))
 (segment (start 149.5 81.5) (end 149.5 80.37) (width 0.254) (layer "B.Cu") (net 6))
 (segment (start 159.52 78) (end 160.02 77.5) (width 0.254) (layer "B.Cu") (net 6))
 (segment (start 123.19 93.98) (end 123.19 88.07) (width 0.254) (layer "B.Cu") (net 6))
 (segment (start 130.81 95.25) (end 124.46 95.25) (width 0.254) (layer "B.Cu") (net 6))
 (segment (start 123.19 76.2) (end 123.19 80.99) (width 0.254) (layer "B.Cu") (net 6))
 (segment (start 123.19 88.07) (end 123.48 87.78) (width 0.254) (layer "B.Cu") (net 6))
 (segment (start 194.945 68.147494) (end 194.945 74.295) (width 0.254) (layer "F.Cu") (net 14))
 (segment (start 200.025 62.865) (end 200.025 63.067494) (width 0.254) (layer "F.Cu") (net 14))
 (segment (start 200.025 63.067494) (end 194.945 68.147494) (width 0.254) (layer "F.Cu") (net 14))
 (via (at 194.945 74.295) (size 0.6) (drill 0.3) (layers "F.Cu" "B.Cu") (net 14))
 (via (at 200.025 62.865) (size 0.6) (drill 0.3) (layers "F.Cu" "B.Cu") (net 14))
 (segment (start 200.66 62.23) (end 200.025 62.865) (width 0.254) (layer "B.Cu") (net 14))
 (segment (start 215.9 50.8) (end 213.995 50.8) (width 0.254) (layer "B.Cu") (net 14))
 (segment (start 194.945 74.295) (end 194.945 82.169) (width 0.254) (layer "B.Cu") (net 14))
 (segment (start 205.105 59.69) (end 203.2 59.69) (width 0.254) (layer "B.Cu") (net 14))
 (segment (start 203.2 59.69) (end 200.66 62.23) (width 0.254) (layer "B.Cu") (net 14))
 (segment (start 194.945 82.169) (end 200.66 87.884) (width 0.254) (layer "B.Cu") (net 14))
 (segment (start 213.995 50.8) (end 205.105 59.69) (width 0.254) (layer "B.Cu") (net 14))
 (segment (start 203.962 69.088) (end 207.01 66.04) (width 0.254) (layer "F.Cu") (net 10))
 (segment (start 198.12 69.088) (end 203.962 69.088) (width 0.254) (layer "F.Cu") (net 10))
 (via (at 198.12 69.088) (size 0.6) (drill 0.3) (layers "F.Cu" "B.Cu") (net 10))
 (via (at 207.01 66.04) (size 0.6) (drill 0.3) (layers "F.Cu" "B.Cu") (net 10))
 (segment (start 185.39 90.424) (end 187.96 90.424) (width 0.254) (layer "B.Cu") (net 10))
 (segment (start 212.09 60.96) (end 215.9 60.96) (width 0.254) (layer "B.Cu") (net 10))
 (segment (start 190.5 71.12) (end 190.5 87.884) (width 0.254) (layer "B.Cu") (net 10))
 (segment (start 192.532 69.088) (end 190.5 71.12) (width 0.254) (layer "B.Cu") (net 10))
 (segment (start 198.12 69.088) (end 192.532 69.088) (width 0.254) (layer "B.Cu") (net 10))
 (segment (start 207.01 66.04) (end 212.09 60.96) (width 0.254) (layer "B.Cu") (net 10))
 (segment (start 187.96 90.424) (end 190.5 87.884) (width 0.254) (layer "B.Cu") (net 10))
 (segment (start 194.31 67.818) (end 194.31 62.23) (width 0.254) (layer "F.Cu") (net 2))
 (via (at 194.31 62.23) (size 0.6) (drill 0.3) (layers "F.Cu" "B.Cu") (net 2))
 (via (at 194.31 67.818) (size 0.6) (drill 0.3) (layers "F.Cu" "B.Cu") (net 2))
 (segment (start 185.39 72.644) (end 187.96 70.074) (width 0.254) (layer "B.Cu") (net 2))
 (segment (start 188.722 67.818) (end 187.96 68.58) (width 0.254) (layer "B.Cu") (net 2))
 (segment (start 194.31 67.818) (end 188.722 67.818) (width 0.254) (layer "B.Cu") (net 2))
 (segment (start 194.31 62.23) (end 194.31 58.42) (width 0.254) (layer "B.Cu") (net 2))
 (segment (start 187.96 68.58) (end 187.96 70.074) (width 0.254) (layer "B.Cu") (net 2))
 (segment (start 191.77 68.58) (end 191.77 62.23) (width 0.254) (layer "F.Cu") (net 3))
 (via (at 191.77 68.58) (size 0.6) (drill 0.3) (layers "F.Cu" "B.Cu") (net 3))
 (via (at 191.77 62.23) (size 0.6) (drill 0.3) (layers "F.Cu" "B.Cu") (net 3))
 (segment (start 189.23 69.85) (end 190.5 68.58) (width 0.254) (layer "B.Cu") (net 3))
 (segment (start 189.23 73.66) (end 189.23 69.85) (width 0.254) (layer "B.Cu") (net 3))
 (segment (start 190.5 68.58) (end 191.77 68.58) (width 0.254) (layer "B.Cu") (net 3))
 (segment (start 187.706 75.184) (end 189.23 73.66) (width 0.254) (layer "B.Cu") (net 3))
 (segment (start 191.77 58.42) (end 191.77 62.23) (width 0.254) (layer "B.Cu") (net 3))
 (segment (start 185.39 75.184) (end 187.706 75.184) (width 0.254) (layer "B.Cu") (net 3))
 (segment (start 208.28 73.66) (end 208.28 82) (width 0.254) (layer "F.Cu") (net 13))
 (via (at 208.28 82) (size 0.6) (drill 0.3) (layers "F.Cu" "B.Cu") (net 13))
 (via (at 208.28 73.66) (size 0.6) (drill 0.3) (layers "F.Cu" "B.Cu") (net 13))
 (segment (start 203.2 60.96) (end 201.93 62.23) (width 0.254) (layer "B.Cu") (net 13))
 (segment (start 201.93 63.5) (end 201.93 67.31) (width 0.254) (layer "B.Cu") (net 13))
 (segment (start 205.74 71.12) (end 208.28 73.66) (width 0.254) (layer "B.Cu") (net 13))
 (segment (start 215.9 53.34) (end 213.36 53.34) (width 0.254) (layer "B.Cu") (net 13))
 (segment (start 213.36 53.34) (end 205.74 60.96) (width 0.254) (layer "B.Cu") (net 13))
 (segment (start 205.74 60.96) (end 203.2 60.96) (width 0.254) (layer "B.Cu") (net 13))
 (segment (start 201.93 67.31) (end 205.74 71.12) (width 0.254) (layer "B.Cu") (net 13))
 (segment (start 200.66 90.424) (end 207.899 90.424) (width 0.254) (layer "B.Cu") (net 13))
 (segment (start 201.93 62.23) (end 201.93 63.5) (width 0.254) (layer "B.Cu") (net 13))
 (segment (start 208.28 90.043) (end 208.28 82) (width 0.254) (layer "B.Cu") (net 13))
 (segment (start 207.899 90.424) (end 208.28 90.043) (width 0.254) (layer "B.Cu") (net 13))
 (segment (start 207.01 92.71) (end 207.01 95.25) (width 0.254) (layer "F.Cu") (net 11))
 (segment (start 210.82 73.66) (end 210.82 82) (width 0.254) (layer "F.Cu") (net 11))
 (via (at 210.82 73.66) (size 0.6) (drill 0.3) (layers "F.Cu" "B.Cu") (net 11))
 (via (at 207.01 92.71) (size 0.6) (drill 0.3) (layers "F.Cu" "B.Cu") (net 11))
 (via (at 210.82 82) (size 0.6) (drill 0.3) (layers "F.Cu" "B.Cu") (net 11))
 (via (at 207.01 95.25) (size 0.6) (drill 0.3) (layers "F.Cu" "B.Cu") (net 11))
 (segment (start 200.66 92.964) (end 201.676 93.98) (width 0.254) (layer "B.Cu") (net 11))
 (segment (start 210.82 60.96) (end 208.28 63.5) (width 0.254) (layer "B.Cu") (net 11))
 (segment (start 206.328 69.168) (end 210.82 73.66) (width 0.254) (layer "B.Cu") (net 11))
 (segment (start 213.36 58.42) (end 210.82 60.96) (width 0.254) (layer "B.Cu") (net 11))
 (segment (start 206.328 65.452) (end 206.328 69.168) (width 0.254) (layer "B.Cu") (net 11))
 (segment (start 210.82 91.44) (end 209.55 92.71) (width 0.254) (layer "B.Cu") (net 11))
 (segment (start 208.28 63.5) (end 206.328 65.452) (width 0.254) (layer "B.Cu") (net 11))
 (segment (start 210.82 82) (end 210.82 91.44) (width 0.254) (layer "B.Cu") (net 11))
 (segment (start 201.676 93.98) (end 203.2 93.98) (width 0.254) (layer "B.Cu") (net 11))
 (segment (start 207.01 95.25) (end 204.47 95.25) (width 0.254) (layer "B.Cu") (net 11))
 (segment (start 209.55 92.71) (end 207.01 92.71) (width 0.254) (layer "B.Cu") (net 11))
 (segment (start 215.9 58.42) (end 213.36 58.42) (width 0.254) (layer "B.Cu") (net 11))
 (segment (start 204.47 95.25) (end 203.2 93.98) (width 0.254) (layer "B.Cu") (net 11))
 (segment (start 209.55 73.66) (end 209.55 82) (width 0.254) (layer "F.Cu") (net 12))
 (segment (start 209.55 91.44) (end 209.55 95.25) (width 0.254) (layer "F.Cu") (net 12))
 (via (at 209.55 73.66) (size 0.6) (drill 0.3) (layers "F.Cu" "B.Cu") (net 12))
 (via (at 209.55 91.44) (size 0.6) (drill 0.3) (layers "F.Cu" "B.Cu") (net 12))
 (via (at 209.55 82) (size 0.6) (drill 0.3) (layers "F.Cu" "B.Cu") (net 12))
 (via (at 209.55 95.25) (size 0.6) (drill 0.3) (layers "F.Cu" "B.Cu") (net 12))
 (segment (start 201.422 96.266) (end 208.534 96.266) (width 0.254) (layer "B.Cu") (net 12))
 (segment (start 200.66 95.504) (end 201.422 96.266) (width 0.254) (layer "B.Cu") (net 12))
 (segment (start 205.74 64.77) (end 205.74 69.85) (width 0.254) (layer "B.Cu") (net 12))
 (segment (start 209.55 82) (end 209.55 91.44) (width 0.254) (layer "B.Cu") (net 12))
 (segment (start 214.63 55.88) (end 205.74 64.77) (width 0.254) (layer "B.Cu") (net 12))
 (segment (start 205.74 69.85) (end 209.55 73.66) (width 0.254) (layer "B.Cu") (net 12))
 (segment (start 208.534 96.266) (end 209.55 95.25) (width 0.254) (layer "B.Cu") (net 12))
 (segment (start 215.9 55.88) (end 214.63 55.88) (width 0.254) (layer "B.Cu") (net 12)))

